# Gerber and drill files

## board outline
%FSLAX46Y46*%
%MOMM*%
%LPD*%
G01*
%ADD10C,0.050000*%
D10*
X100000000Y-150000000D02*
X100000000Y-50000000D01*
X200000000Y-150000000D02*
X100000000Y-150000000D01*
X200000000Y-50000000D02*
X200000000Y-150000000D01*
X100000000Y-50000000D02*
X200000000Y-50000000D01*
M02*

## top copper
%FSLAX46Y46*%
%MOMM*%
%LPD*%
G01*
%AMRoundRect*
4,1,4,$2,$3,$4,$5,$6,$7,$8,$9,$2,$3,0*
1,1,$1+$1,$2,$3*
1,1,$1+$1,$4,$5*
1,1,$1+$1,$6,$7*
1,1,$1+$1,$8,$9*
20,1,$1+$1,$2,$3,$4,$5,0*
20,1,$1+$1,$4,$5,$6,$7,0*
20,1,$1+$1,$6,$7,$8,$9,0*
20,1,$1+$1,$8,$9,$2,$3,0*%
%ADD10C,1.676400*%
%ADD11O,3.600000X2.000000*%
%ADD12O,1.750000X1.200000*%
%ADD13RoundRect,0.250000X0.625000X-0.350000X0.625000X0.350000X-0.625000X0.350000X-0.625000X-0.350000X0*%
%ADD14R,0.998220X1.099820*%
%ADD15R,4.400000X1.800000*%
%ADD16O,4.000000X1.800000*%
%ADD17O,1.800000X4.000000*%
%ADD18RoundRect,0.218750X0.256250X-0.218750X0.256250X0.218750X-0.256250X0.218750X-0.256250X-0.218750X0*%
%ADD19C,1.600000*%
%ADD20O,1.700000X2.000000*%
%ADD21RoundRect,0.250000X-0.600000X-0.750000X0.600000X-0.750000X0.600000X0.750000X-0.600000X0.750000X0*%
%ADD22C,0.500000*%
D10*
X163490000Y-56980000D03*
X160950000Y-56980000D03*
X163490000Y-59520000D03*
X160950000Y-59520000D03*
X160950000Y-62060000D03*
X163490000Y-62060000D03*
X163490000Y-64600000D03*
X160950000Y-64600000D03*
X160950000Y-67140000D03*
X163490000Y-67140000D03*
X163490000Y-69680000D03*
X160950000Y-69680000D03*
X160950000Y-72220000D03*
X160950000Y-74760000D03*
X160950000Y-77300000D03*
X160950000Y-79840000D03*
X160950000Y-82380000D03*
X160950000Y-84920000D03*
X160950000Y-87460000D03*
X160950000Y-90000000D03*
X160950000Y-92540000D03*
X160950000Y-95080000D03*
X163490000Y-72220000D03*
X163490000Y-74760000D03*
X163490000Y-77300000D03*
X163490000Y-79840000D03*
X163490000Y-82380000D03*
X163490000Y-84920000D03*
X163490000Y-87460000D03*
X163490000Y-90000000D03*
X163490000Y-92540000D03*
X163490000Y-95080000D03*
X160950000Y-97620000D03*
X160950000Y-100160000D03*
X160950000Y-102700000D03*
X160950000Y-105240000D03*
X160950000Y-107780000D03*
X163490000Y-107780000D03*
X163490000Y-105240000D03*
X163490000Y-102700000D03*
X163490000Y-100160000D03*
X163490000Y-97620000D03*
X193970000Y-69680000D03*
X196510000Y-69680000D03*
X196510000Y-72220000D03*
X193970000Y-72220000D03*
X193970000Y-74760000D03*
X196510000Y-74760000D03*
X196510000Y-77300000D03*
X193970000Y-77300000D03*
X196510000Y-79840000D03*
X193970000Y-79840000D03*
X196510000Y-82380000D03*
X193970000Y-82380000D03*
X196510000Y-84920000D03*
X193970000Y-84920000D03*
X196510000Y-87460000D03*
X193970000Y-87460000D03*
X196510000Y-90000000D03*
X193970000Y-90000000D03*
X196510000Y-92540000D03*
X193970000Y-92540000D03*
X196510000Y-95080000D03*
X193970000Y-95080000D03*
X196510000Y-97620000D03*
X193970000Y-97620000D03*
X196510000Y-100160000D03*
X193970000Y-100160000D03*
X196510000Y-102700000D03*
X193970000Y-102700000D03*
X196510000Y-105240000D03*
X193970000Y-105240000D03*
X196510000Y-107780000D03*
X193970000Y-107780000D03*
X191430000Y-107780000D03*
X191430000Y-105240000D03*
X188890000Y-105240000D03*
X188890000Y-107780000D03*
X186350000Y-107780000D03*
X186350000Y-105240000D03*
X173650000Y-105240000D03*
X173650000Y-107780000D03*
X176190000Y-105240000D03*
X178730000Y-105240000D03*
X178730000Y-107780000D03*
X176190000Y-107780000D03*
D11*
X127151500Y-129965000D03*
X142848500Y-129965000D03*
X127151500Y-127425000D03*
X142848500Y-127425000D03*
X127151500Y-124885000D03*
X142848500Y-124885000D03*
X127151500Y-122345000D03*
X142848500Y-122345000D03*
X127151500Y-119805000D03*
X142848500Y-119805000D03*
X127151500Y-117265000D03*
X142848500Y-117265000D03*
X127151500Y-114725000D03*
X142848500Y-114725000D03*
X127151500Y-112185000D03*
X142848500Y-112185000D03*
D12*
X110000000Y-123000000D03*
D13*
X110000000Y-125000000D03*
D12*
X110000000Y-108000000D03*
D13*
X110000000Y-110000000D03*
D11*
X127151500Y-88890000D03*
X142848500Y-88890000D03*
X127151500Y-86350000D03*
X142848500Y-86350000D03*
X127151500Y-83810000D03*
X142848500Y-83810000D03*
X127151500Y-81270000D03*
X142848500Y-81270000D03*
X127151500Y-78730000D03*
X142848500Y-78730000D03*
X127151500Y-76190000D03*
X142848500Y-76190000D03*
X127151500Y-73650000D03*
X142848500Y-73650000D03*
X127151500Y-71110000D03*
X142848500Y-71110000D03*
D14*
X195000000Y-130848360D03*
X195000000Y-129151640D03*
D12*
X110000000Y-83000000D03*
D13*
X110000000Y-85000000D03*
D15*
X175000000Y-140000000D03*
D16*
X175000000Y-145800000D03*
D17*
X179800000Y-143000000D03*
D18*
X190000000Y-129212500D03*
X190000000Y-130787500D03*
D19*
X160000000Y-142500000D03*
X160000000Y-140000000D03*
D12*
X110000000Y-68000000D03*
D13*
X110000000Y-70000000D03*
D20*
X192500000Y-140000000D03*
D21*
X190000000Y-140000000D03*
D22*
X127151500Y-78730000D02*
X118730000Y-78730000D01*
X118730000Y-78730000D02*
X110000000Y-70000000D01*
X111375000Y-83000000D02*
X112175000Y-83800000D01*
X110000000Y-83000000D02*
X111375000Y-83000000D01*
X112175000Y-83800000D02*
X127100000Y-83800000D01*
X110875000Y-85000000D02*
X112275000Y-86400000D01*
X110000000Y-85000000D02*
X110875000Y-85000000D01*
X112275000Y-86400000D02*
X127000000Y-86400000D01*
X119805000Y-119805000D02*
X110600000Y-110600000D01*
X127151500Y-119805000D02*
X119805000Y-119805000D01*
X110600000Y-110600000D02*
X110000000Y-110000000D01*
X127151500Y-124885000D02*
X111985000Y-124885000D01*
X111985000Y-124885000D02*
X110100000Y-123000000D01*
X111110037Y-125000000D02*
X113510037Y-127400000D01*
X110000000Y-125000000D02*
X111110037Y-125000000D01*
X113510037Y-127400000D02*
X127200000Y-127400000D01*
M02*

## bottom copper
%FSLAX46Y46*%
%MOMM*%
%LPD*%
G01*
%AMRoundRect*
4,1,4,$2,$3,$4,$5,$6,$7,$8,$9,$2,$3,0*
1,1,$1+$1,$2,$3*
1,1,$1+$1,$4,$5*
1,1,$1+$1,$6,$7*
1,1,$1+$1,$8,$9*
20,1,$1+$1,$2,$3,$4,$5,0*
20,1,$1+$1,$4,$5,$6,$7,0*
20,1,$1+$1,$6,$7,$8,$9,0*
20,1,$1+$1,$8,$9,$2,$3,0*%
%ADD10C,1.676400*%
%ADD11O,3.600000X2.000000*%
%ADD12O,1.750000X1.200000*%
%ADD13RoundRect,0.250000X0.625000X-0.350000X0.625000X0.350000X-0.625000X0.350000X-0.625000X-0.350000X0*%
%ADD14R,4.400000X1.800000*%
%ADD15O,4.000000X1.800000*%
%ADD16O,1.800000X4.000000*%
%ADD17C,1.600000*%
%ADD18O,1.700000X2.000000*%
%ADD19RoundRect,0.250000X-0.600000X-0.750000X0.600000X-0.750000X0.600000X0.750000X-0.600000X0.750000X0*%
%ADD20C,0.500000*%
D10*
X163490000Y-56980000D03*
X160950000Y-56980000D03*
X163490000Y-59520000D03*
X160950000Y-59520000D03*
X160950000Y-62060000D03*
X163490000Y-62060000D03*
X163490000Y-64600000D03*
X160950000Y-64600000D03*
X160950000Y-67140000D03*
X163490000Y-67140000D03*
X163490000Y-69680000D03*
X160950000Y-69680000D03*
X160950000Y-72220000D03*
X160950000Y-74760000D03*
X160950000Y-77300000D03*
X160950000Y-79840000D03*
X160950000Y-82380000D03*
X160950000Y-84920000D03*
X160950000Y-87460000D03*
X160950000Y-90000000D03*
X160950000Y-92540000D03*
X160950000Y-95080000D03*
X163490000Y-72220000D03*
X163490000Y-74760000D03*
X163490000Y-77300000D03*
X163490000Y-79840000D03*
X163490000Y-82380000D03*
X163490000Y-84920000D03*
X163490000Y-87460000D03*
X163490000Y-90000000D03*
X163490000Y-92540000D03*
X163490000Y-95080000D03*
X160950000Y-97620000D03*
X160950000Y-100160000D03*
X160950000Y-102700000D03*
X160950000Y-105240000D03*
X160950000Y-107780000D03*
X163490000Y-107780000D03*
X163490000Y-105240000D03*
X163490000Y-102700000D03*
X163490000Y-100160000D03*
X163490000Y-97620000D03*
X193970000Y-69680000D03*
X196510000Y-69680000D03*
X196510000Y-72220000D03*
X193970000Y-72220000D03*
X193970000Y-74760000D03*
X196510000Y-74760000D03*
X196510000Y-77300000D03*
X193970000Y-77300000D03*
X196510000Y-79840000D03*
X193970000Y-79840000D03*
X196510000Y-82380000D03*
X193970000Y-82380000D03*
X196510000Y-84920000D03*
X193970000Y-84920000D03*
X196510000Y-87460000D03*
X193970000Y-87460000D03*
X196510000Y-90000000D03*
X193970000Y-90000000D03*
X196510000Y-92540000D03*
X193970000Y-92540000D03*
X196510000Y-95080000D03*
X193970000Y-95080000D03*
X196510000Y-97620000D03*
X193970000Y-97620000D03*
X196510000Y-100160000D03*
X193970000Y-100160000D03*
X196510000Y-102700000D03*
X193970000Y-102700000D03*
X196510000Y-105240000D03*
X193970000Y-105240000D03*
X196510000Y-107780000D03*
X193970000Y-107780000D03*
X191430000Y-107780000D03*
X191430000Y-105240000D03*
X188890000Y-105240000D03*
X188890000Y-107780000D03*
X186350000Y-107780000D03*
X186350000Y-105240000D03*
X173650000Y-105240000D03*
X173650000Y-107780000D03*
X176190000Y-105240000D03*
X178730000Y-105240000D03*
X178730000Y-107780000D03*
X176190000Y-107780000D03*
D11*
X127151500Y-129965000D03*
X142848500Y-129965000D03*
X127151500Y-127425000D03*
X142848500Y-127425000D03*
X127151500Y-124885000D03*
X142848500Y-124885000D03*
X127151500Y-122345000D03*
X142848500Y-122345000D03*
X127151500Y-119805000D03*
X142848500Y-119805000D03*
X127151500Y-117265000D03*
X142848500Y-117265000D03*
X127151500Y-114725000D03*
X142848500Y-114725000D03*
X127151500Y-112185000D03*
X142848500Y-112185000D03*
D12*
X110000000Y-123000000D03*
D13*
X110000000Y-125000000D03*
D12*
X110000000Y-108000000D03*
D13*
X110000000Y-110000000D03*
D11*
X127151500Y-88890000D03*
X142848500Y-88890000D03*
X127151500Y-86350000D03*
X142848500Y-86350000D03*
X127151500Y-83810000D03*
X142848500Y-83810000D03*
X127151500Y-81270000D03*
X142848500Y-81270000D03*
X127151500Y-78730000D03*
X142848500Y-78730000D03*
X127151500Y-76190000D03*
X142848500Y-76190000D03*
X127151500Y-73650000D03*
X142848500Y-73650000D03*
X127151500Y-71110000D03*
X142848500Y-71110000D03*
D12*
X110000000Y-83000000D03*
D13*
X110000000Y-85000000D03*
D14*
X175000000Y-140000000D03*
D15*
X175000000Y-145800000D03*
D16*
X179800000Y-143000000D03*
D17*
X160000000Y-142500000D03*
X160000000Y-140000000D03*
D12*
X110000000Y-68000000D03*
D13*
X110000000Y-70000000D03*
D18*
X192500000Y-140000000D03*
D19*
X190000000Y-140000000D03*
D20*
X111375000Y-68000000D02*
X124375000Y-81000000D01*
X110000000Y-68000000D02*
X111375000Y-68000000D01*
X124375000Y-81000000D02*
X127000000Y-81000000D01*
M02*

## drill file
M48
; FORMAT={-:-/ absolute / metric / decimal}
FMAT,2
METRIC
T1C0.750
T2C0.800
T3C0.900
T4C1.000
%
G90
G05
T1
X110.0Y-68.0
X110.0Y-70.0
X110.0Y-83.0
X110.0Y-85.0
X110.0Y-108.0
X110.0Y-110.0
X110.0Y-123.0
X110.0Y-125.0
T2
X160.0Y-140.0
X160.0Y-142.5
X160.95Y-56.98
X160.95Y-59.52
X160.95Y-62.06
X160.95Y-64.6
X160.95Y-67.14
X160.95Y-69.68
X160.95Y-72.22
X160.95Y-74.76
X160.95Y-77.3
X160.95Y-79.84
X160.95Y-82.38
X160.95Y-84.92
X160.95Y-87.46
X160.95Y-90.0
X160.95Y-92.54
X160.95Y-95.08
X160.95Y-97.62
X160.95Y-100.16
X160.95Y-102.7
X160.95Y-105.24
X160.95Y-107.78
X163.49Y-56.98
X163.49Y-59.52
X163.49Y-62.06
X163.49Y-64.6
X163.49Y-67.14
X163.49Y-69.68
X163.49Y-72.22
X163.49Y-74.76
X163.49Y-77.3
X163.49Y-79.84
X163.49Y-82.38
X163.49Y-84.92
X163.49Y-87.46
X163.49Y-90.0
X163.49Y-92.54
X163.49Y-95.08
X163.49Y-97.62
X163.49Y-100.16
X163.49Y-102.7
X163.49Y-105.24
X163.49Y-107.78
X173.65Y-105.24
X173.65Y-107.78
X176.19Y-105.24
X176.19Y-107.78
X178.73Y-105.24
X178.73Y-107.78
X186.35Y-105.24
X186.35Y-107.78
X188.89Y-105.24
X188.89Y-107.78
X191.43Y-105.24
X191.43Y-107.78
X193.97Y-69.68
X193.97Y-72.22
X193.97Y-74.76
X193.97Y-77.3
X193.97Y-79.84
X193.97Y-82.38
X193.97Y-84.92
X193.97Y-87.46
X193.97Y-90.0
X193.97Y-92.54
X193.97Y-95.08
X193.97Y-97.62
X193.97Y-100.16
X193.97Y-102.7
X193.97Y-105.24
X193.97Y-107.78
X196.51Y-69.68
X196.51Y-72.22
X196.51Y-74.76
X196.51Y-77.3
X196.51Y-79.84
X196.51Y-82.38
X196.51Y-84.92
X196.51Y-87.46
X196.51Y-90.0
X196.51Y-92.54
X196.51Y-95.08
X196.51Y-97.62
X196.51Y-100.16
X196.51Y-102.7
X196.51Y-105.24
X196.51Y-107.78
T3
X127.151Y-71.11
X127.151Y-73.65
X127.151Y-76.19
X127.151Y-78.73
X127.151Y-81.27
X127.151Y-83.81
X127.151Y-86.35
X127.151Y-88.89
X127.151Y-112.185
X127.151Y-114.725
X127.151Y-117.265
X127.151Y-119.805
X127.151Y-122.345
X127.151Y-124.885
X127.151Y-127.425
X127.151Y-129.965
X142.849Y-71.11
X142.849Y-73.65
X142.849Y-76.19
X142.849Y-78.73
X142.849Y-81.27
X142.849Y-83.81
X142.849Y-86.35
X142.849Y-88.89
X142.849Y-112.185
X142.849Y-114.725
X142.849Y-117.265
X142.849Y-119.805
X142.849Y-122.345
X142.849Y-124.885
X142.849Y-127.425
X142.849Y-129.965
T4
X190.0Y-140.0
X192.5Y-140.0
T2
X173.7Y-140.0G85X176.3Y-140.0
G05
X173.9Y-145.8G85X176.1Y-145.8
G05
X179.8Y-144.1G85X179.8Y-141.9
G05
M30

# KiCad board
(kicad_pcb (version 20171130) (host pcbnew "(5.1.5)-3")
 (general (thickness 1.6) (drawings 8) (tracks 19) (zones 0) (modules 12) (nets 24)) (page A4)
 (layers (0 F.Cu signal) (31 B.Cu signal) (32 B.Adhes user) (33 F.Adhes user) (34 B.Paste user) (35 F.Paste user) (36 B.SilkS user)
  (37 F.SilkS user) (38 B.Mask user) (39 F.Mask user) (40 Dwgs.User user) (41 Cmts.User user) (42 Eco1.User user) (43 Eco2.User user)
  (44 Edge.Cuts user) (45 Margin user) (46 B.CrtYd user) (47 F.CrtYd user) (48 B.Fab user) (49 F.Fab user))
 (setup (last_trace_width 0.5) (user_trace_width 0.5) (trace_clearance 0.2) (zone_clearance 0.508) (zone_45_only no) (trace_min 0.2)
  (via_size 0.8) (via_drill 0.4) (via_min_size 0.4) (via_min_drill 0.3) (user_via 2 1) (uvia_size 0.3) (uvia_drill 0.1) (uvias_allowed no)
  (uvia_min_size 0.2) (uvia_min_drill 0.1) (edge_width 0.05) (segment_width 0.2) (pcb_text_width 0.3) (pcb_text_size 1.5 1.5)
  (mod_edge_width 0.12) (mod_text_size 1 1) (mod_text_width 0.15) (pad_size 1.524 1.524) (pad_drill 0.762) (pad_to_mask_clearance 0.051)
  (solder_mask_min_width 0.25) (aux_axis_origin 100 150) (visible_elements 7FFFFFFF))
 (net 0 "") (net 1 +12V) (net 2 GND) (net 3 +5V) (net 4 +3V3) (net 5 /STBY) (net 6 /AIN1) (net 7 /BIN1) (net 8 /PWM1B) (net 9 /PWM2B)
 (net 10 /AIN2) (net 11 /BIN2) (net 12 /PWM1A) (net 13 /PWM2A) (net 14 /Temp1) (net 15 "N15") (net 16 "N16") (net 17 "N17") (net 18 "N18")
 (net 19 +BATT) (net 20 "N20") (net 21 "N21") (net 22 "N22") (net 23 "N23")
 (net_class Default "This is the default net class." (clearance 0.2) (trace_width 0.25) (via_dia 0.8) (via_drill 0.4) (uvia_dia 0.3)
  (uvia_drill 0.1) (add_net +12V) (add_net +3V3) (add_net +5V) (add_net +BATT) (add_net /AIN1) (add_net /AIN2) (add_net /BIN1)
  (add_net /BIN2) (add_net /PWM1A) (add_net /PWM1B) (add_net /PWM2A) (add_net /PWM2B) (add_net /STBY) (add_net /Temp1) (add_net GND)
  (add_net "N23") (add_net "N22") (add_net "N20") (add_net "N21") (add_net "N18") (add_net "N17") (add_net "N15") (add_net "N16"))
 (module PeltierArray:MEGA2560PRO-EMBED (layer F.Cu) (at 180 90 270)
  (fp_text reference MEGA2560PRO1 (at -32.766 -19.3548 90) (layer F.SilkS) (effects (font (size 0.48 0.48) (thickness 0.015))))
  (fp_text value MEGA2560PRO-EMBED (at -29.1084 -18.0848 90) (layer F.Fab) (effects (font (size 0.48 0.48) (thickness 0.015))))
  (pad VIN@2 thru_hole circle (at -33.02 16.51 270) (size 1.6764 1.6764) (drill 0.8) (layers *.Cu *.Mask) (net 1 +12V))
  (pad VIN@1 thru_hole circle (at -33.02 19.05 270) (size 1.6764 1.6764) (drill 0.8) (layers *.Cu *.Mask) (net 1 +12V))
  (pad GND@2 thru_hole circle (at -30.48 16.51 270) (size 1.6764 1.6764) (drill 0.8) (layers *.Cu *.Mask) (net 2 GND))
  (pad GND@1 thru_hole circle (at -30.48 19.05 270) (size 1.6764 1.6764) (drill 0.8) (layers *.Cu *.Mask) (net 2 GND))
  (pad 5V@1 thru_hole circle (at -27.94 19.05 270) (size 1.6764 1.6764) (drill 0.8) (layers *.Cu *.Mask) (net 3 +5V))
  (pad 5V@2 thru_hole circle (at -27.94 16.51 270) (size 1.6764 1.6764) (drill 0.8) (layers *.Cu *.Mask) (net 3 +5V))
  (pad 3V3@2 thru_hole circle (at -25.4 16.51 270) (size 1.6764 1.6764) (drill 0.8) (layers *.Cu *.Mask) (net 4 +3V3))
  (pad 3V3@1 thru_hole circle (at -25.4 19.05 270) (size 1.6764 1.6764) (drill 0.8) (layers *.Cu *.Mask) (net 4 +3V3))
  (pad RST thru_hole circle (at -22.86 19.05 270) (size 1.6764 1.6764) (drill 0.8) (layers *.Cu *.Mask))
  (pad AREF thru_hole circle (at -22.86 16.51 270) (size 1.6764 1.6764) (drill 0.8) (layers *.Cu *.Mask))
  (pad RX thru_hole circle (at -20.32 16.51 270) (size 1.6764 1.6764) (drill 0.8) (layers *.Cu *.Mask))
  (pad TX thru_hole circle (at -20.32 19.05 270) (size 1.6764 1.6764) (drill 0.8) (layers *.Cu *.Mask))
  (pad D3 thru_hole circle (at -17.78 19.05 270) (size 1.6764 1.6764) (drill 0.8) (layers *.Cu *.Mask) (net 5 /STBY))
  (pad D5 thru_hole circle (at -15.24 19.05 270) (size 1.6764 1.6764) (drill 0.8) (layers *.Cu *.Mask) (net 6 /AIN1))
  (pad D7 thru_hole circle (at -12.7 19.05 270) (size 1.6764 1.6764) (drill 0.8) (layers *.Cu *.Mask) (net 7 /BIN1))
  (pad D9 thru_hole circle (at -10.16 19.05 270) (size 1.6764 1.6764) (drill 0.8) (layers *.Cu *.Mask) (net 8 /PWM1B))
  (pad D11 thru_hole circle (at -7.62 19.05 270) (size 1.6764 1.6764) (drill 0.8) (layers *.Cu *.Mask) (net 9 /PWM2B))
  (pad D13 thru_hole circle (at -5.08 19.05 270) (size 1.6764 1.6764) (drill 0.8) (layers *.Cu *.Mask))
  (pad D15 thru_hole circle (at -2.54 19.05 270) (size 1.6764 1.6764) (drill 0.8) (layers *.Cu *.Mask))
  (pad D17 thru_hole circle (at 0 19.05 270) (size 1.6764 1.6764) (drill 0.8) (layers *.Cu *.Mask))
  (pad D19 thru_hole circle (at 2.54 19.05 270) (size 1.6764 1.6764) (drill 0.8) (layers *.Cu *.Mask))
  (pad D21 thru_hole circle (at 5.08 19.05 270) (size 1.6764 1.6764) (drill 0.8) (layers *.Cu *.Mask))
  (pad D2 thru_hole circle (at -17.78 16.51 270) (size 1.6764 1.6764) (drill 0.8) (layers *.Cu *.Mask))
  (pad D4 thru_hole circle (at -15.24 16.51 270) (size 1.6764 1.6764) (drill 0.8) (layers *.Cu *.Mask) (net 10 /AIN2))
  (pad D6 thru_hole circle (at -12.7 16.51 270) (size 1.6764 1.6764) (drill 0.8) (layers *.Cu *.Mask) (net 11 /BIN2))
  (pad D8 thru_hole circle (at -10.16 16.51 270) (size 1.6764 1.6764) (drill 0.8) (layers *.Cu *.Mask) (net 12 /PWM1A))
  (pad D10 thru_hole circle (at -7.62 16.51 270) (size 1.6764 1.6764) (drill 0.8) (layers *.Cu *.Mask) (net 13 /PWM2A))
  (pad D12 thru_hole circle (at -5.08 16.51 270) (size 1.6764 1.6764) (drill 0.8) (layers *.Cu *.Mask))
  (pad D14 thru_hole circle (at -2.54 16.51 270) (size 1.6764 1.6764) (drill 0.8) (layers *.Cu *.Mask))
  (pad D16 thru_hole circle (at 0 16.51 270) (size 1.6764 1.6764) (drill 0.8) (layers *.Cu *.Mask))
  (pad D18 thru_hole circle (at 2.54 16.51 270) (size 1.6764 1.6764) (drill 0.8) (layers *.Cu *.Mask))
  (pad D20 thru_hole circle (at 5.08 16.51 270) (size 1.6764 1.6764) (drill 0.8) (layers *.Cu *.Mask))
  (pad D23 thru_hole circle (at 7.62 19.05 270) (size 1.6764 1.6764) (drill 0.8) (layers *.Cu *.Mask))
  (pad D25 thru_hole circle (at 10.16 19.05 270) (size 1.6764 1.6764) (drill 0.8) (layers *.Cu *.Mask))
  (pad D27 thru_hole circle (at 12.7 19.05 270) (size 1.6764 1.6764) (drill 0.8) (layers *.Cu *.Mask))
  (pad D29 thru_hole circle (at 15.24 19.05 270) (size 1.6764 1.6764) (drill 0.8) (layers *.Cu *.Mask))
  (pad D31 thru_hole circle (at 17.78 19.05 270) (size 1.6764 1.6764) (drill 0.8) (layers *.Cu *.Mask))
  (pad D30 thru_hole circle (at 17.78 16.51 270) (size 1.6764 1.6764) (drill 0.8) (layers *.Cu *.Mask))
  (pad D28 thru_hole circle (at 15.24 16.51 270) (size 1.6764 1.6764) (drill 0.8) (layers *.Cu *.Mask))
  (pad D26 thru_hole circle (at 12.7 16.51 270) (size 1.6764 1.6764) (drill 0.8) (layers *.Cu *.Mask))
  (pad D24 thru_hole circle (at 10.16 16.51 270) (size 1.6764 1.6764) (drill 0.8) (layers *.Cu *.Mask))
  (pad D22 thru_hole circle (at 7.62 16.51 270) (size 1.6764 1.6764) (drill 0.8) (layers *.Cu *.Mask))
  (pad A1 thru_hole circle (at -20.32 -13.97 270) (size 1.6764 1.6764) (drill 0.8) (layers *.Cu *.Mask))
  (pad A0 thru_hole circle (at -20.32 -16.51 270) (size 1.6764 1.6764) (drill 0.8) (layers *.Cu *.Mask) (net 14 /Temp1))
  (pad A2 thru_hole circle (at -17.78 -16.51 270) (size 1.6764 1.6764) (drill 0.8) (layers *.Cu *.Mask))
  (pad A3 thru_hole circle (at -17.78 -13.97 270) (size 1.6764 1.6764) (drill 0.8) (layers *.Cu *.Mask))
  (pad A5 thru_hole circle (at -15.24 -13.97 270) (size 1.6764 1.6764) (drill 0.8) (layers *.Cu *.Mask))
  (pad A4 thru_hole circle (at -15.24 -16.51 270) (size 1.6764 1.6764) (drill 0.8) (layers *.Cu *.Mask))
  (pad A6 thru_hole circle (at -12.7 -16.51 270) (size 1.6764 1.6764) (drill 0.8) (layers *.Cu *.Mask))
  (pad A7 thru_hole circle (at -12.7 -13.97 270) (size 1.6764 1.6764) (drill 0.8) (layers *.Cu *.Mask))
  (pad A8 thru_hole circle (at -10.16 -16.51 270) (size 1.6764 1.6764) (drill 0.8) (layers *.Cu *.Mask))
  (pad A9 thru_hole circle (at -10.16 -13.97 270) (size 1.6764 1.6764) (drill 0.8) (layers *.Cu *.Mask))
  (pad A10 thru_hole circle (at -7.62 -16.51 270) (size 1.6764 1.6764) (drill 0.8) (layers *.Cu *.Mask))
  (pad A11 thru_hole circle (at -7.62 -13.97 270) (size 1.6764 1.6764) (drill 0.8) (layers *.Cu *.Mask))
  (pad A12 thru_hole circle (at -5.08 -16.51 270) (size 1.6764 1.6764) (drill 0.8) (layers *.Cu *.Mask))
  (pad A13 thru_hole circle (at -5.08 -13.97 270) (size 1.6764 1.6764) (drill 0.8) (layers *.Cu *.Mask))
  (pad A14 thru_hole circle (at -2.54 -16.51 270) (size 1.6764 1.6764) (drill 0.8) (layers *.Cu *.Mask))
  (pad A15 thru_hole circle (at -2.54 -13.97 270) (size 1.6764 1.6764) (drill 0.8) (layers *.Cu *.Mask))
  (pad D32 thru_hole circle (at 0 -16.51 270) (size 1.6764 1.6764) (drill 0.8) (layers *.Cu *.Mask))
  (pad D33 thru_hole circle (at 0 -13.97 270) (size 1.6764 1.6764) (drill 0.8) (layers *.Cu *.Mask))
  (pad D34 thru_hole circle (at 2.54 -16.51 270) (size 1.6764 1.6764) (drill 0.8) (layers *.Cu *.Mask))
  (pad D35 thru_hole circle (at 2.54 -13.97 270) (size 1.6764 1.6764) (drill 0.8) (layers *.Cu *.Mask))
  (pad D36 thru_hole circle (at 5.08 -16.51 270) (size 1.6764 1.6764) (drill 0.8) (layers *.Cu *.Mask))
  (pad D37 thru_hole circle (at 5.08 -13.97 270) (size 1.6764 1.6764) (drill 0.8) (layers *.Cu *.Mask))
  (pad D38 thru_hole circle (at 7.62 -16.51 270) (size 1.6764 1.6764) (drill 0.8) (layers *.Cu *.Mask))
  (pad D39 thru_hole circle (at 7.62 -13.97 270) (size 1.6764 1.6764) (drill 0.8) (layers *.Cu *.Mask))
  (pad D40 thru_hole circle (at 10.16 -16.51 270) (size 1.6764 1.6764) (drill 0.8) (layers *.Cu *.Mask))
  (pad D41 thru_hole circle (at 10.16 -13.97 270) (size 1.6764 1.6764) (drill 0.8) (layers *.Cu *.Mask))
  (pad D42 thru_hole circle (at 12.7 -16.51 270) (size 1.6764 1.6764) (drill 0.8) (layers *.Cu *.Mask))
  (pad D43 thru_hole circle (at 12.7 -13.97 270) (size 1.6764 1.6764) (drill 0.8) (layers *.Cu *.Mask))
  (pad D44 thru_hole circle (at 15.24 -16.51 270) (size 1.6764 1.6764) (drill 0.8) (layers *.Cu *.Mask))
  (pad D45 thru_hole circle (at 15.24 -13.97 270) (size 1.6764 1.6764) (drill 0.8) (layers *.Cu *.Mask))
  (pad D46 thru_hole circle (at 17.78 -16.51 270) (size 1.6764 1.6764) (drill 0.8) (layers *.Cu *.Mask))
  (pad D47 thru_hole circle (at 17.78 -13.97 270) (size 1.6764 1.6764) (drill 0.8) (layers *.Cu *.Mask))
  (pad D48 thru_hole circle (at 17.78 -11.43 270) (size 1.6764 1.6764) (drill 0.8) (layers *.Cu *.Mask))
  (pad D49 thru_hole circle (at 15.24 -11.43 270) (size 1.6764 1.6764) (drill 0.8) (layers *.Cu *.Mask))
  (pad D51 thru_hole circle (at 15.24 -8.89 270) (size 1.6764 1.6764) (drill 0.8) (layers *.Cu *.Mask))
  (pad D50 thru_hole circle (at 17.78 -8.89 270) (size 1.6764 1.6764) (drill 0.8) (layers *.Cu *.Mask))
  (pad D52 thru_hole circle (at 17.78 -6.35 270) (size 1.6764 1.6764) (drill 0.8) (layers *.Cu *.Mask))
  (pad D53 thru_hole circle (at 15.24 -6.35 270) (size 1.6764 1.6764) (drill 0.8) (layers *.Cu *.Mask))
  (pad RESET thru_hole circle (at 15.24 6.35 270) (size 1.6764 1.6764) (drill 0.8) (layers *.Cu *.Mask))
  (pad GND@3 thru_hole circle (at 17.78 6.35 270) (size 1.6764 1.6764) (drill 0.8) (layers *.Cu *.Mask) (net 2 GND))
  (pad SCK thru_hole circle (at 15.24 3.81 270) (size 1.6764 1.6764) (drill 0.8) (layers *.Cu *.Mask))
  (pad MISO thru_hole circle (at 15.24 1.27 270) (size 1.6764 1.6764) (drill 0.8) (layers *.Cu *.Mask))
  (pad 5V@3 thru_hole circle (at 17.78 1.27 270) (size 1.6764 1.6764) (drill 0.8) (layers *.Cu *.Mask) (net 3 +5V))
  (pad MOSI thru_hole circle (at 17.78 3.81 270) (size 1.6764 1.6764) (drill 0.8) (layers *.Cu *.Mask)))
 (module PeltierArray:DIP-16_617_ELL (layer F.Cu) (at 135 121.075 270)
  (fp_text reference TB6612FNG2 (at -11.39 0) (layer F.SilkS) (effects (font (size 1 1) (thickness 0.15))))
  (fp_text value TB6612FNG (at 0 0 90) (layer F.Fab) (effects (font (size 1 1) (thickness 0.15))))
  (pad 8 thru_hole oval (at 8.89 7.8485 270) (size 2 3.6) (drill 0.9) (layers *.Cu *.Mask) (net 2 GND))
  (pad 9 thru_hole oval (at 8.89 -7.8485 270) (size 2 3.6) (drill 0.9) (layers *.Cu *.Mask) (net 13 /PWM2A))
  (pad 7 thru_hole oval (at 6.35 7.8485 270) (size 2 3.6) (drill 0.9) (layers *.Cu *.Mask) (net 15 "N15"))
  (pad 10 thru_hole oval (at 6.35 -7.8485 270) (size 2 3.6) (drill 0.9) (layers *.Cu *.Mask) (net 10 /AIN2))
  (pad 6 thru_hole oval (at 3.81 7.8485 270) (size 2 3.6) (drill 0.9) (layers *.Cu *.Mask) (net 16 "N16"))
  (pad 11 thru_hole oval (at 3.81 -7.8485 270) (size 2 3.6) (drill 0.9) (layers *.Cu *.Mask) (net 6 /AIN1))
  (pad 5 thru_hole oval (at 1.27 7.8485 270) (size 2 3.6) (drill 0.9) (layers *.Cu *.Mask) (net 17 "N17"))
  (pad 12 thru_hole oval (at 1.27 -7.8485 270) (size 2 3.6) (drill 0.9) (layers *.Cu *.Mask) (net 5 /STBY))
  (pad 4 thru_hole oval (at -1.27 7.8485 270) (size 2 3.6) (drill 0.9) (layers *.Cu *.Mask) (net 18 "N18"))
  (pad 13 thru_hole oval (at -1.27 -7.8485 270) (size 2 3.6) (drill 0.9) (layers *.Cu *.Mask) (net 7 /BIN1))
  (pad 3 thru_hole oval (at -3.81 7.8485 270) (size 2 3.6) (drill 0.9) (layers *.Cu *.Mask) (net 2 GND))
  (pad 14 thru_hole oval (at -3.81 -7.8485 270) (size 2 3.6) (drill 0.9) (layers *.Cu *.Mask) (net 11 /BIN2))
  (pad 2 thru_hole oval (at -6.35 7.8485 270) (size 2 3.6) (drill 0.9) (layers *.Cu *.Mask) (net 3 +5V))
  (pad 15 thru_hole oval (at -6.35 -7.8485 270) (size 2 3.6) (drill 0.9) (layers *.Cu *.Mask) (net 9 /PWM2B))
  (pad 1 thru_hole oval (at -8.89 7.8485 270) (size 2 3.6) (drill 0.9) (layers *.Cu *.Mask) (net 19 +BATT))
  (pad 16 thru_hole oval (at -8.89 -7.8485 270) (size 2 3.6) (drill 0.9) (layers *.Cu *.Mask) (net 2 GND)))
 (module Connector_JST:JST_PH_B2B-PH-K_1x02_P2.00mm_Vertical (layer F.Cu) (at 110 125 90)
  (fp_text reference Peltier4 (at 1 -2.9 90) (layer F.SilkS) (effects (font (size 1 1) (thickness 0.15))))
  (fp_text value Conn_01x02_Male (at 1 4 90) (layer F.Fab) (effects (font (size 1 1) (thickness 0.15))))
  (pad 2 thru_hole oval (at 2 0 90) (size 1.2 1.75) (drill 0.75) (layers *.Cu *.Mask) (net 16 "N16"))
  (pad 1 thru_hole roundrect (at 0 0 90) (size 1.2 1.75) (drill 0.75) (layers *.Cu *.Mask) (roundrect_rratio 0.208333) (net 15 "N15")))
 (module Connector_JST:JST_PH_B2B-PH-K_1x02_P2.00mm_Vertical (layer F.Cu) (at 110 110 90)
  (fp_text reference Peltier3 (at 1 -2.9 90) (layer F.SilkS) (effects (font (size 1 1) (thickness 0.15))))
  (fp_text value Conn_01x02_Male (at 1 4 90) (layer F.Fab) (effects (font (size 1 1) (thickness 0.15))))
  (pad 2 thru_hole oval (at 2 0 90) (size 1.2 1.75) (drill 0.75) (layers *.Cu *.Mask) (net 17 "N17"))
  (pad 1 thru_hole roundrect (at 0 0 90) (size 1.2 1.75) (drill 0.75) (layers *.Cu *.Mask) (roundrect_rratio 0.208333) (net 18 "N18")))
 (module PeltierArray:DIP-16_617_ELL (layer F.Cu) (at 135 80 270)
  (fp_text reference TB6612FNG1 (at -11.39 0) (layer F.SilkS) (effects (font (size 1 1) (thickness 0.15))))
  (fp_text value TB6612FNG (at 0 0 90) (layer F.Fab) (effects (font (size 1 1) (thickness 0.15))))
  (pad 8 thru_hole oval (at 8.89 7.8485 270) (size 2 3.6) (drill 0.9) (layers *.Cu *.Mask) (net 2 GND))
  (pad 9 thru_hole oval (at 8.89 -7.8485 270) (size 2 3.6) (drill 0.9) (layers *.Cu *.Mask) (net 12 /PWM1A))
  (pad 7 thru_hole oval (at 6.35 7.8485 270) (size 2 3.6) (drill 0.9) (layers *.Cu *.Mask) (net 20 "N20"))
  (pad 10 thru_hole oval (at 6.35 -7.8485 270) (size 2 3.6) (drill 0.9) (layers *.Cu *.Mask) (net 10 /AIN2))
  (pad 6 thru_hole oval (at 3.81 7.8485 270) (size 2 3.6) (drill 0.9) (layers *.Cu *.Mask) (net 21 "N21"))
  (pad 11 thru_hole oval (at 3.81 -7.8485 270) (size 2 3.6) (drill 0.9) (layers *.Cu *.Mask) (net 6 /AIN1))
  (pad 5 thru_hole oval (at 1.27 7.8485 270) (size 2 3.6) (drill 0.9) (layers *.Cu *.Mask) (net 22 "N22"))
  (pad 12 thru_hole oval (at 1.27 -7.8485 270) (size 2 3.6) (drill 0.9) (layers *.Cu *.Mask) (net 5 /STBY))
  (pad 4 thru_hole oval (at -1.27 7.8485 270) (size 2 3.6) (drill 0.9) (layers *.Cu *.Mask) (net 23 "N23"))
  (pad 13 thru_hole oval (at -1.27 -7.8485 270) (size 2 3.6) (drill 0.9) (layers *.Cu *.Mask) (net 7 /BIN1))
  (pad 3 thru_hole oval (at -3.81 7.8485 270) (size 2 3.6) (drill 0.9) (layers *.Cu *.Mask) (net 2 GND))
  (pad 14 thru_hole oval (at -3.81 -7.8485 270) (size 2 3.6) (drill 0.9) (layers *.Cu *.Mask) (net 11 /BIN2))
  (pad 2 thru_hole oval (at -6.35 7.8485 270) (size 2 3.6) (drill 0.9) (layers *.Cu *.Mask) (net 3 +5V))
  (pad 15 thru_hole oval (at -6.35 -7.8485 270) (size 2 3.6) (drill 0.9) (layers *.Cu *.Mask) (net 8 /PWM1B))
  (pad 1 thru_hole oval (at -8.89 7.8485 270) (size 2 3.6) (drill 0.9) (layers *.Cu *.Mask) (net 19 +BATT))
  (pad 16 thru_hole oval (at -8.89 -7.8485 270) (size 2 3.6) (drill 0.9) (layers *.Cu *.Mask) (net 2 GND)))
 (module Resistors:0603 (layer F.Cu) (at 195 130 270)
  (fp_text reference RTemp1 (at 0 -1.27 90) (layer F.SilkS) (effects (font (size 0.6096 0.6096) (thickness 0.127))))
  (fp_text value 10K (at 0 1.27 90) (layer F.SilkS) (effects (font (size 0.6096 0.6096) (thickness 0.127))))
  (pad 2 smd rect (at 0.84836 0 270) (size 1.09982 0.99822) (layers F.Cu F.Paste F.Mask) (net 14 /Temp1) (solder_mask_margin 0.1016))
  (pad 1 smd rect (at -0.84836 0 270) (size 1.09982 0.99822) (layers F.Cu F.Paste F.Mask) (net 2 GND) (solder_mask_margin 0.1016)))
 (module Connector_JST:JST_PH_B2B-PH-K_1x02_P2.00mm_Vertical (layer F.Cu) (at 110 85 90)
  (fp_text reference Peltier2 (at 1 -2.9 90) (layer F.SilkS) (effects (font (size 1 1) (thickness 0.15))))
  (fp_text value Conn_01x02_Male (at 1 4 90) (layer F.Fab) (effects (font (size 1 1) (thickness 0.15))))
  (pad 2 thru_hole oval (at 2 0 90) (size 1.2 1.75) (drill 0.75) (layers *.Cu *.Mask) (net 21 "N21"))
  (pad 1 thru_hole roundrect (at 0 0 90) (size 1.2 1.75) (drill 0.75) (layers *.Cu *.Mask) (roundrect_rratio 0.208333) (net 20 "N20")))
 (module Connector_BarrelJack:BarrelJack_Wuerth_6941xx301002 (layer F.Cu) (at 175 140)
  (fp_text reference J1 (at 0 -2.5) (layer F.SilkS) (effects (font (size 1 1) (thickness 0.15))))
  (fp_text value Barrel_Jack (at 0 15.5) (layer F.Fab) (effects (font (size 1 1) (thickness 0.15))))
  (pad 1 thru_hole rect (at 0 0) (size 4.4 1.8) (drill oval 3.4 0.8) (layers *.Cu *.Mask) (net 19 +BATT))
  (pad 2 thru_hole oval (at 0 5.8) (size 4 1.8) (drill oval 3 0.8) (layers *.Cu *.Mask) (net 2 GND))
  (pad 3 thru_hole oval (at 4.8 3 90) (size 4 1.8) (drill oval 3 0.8) (layers *.Cu *.Mask)))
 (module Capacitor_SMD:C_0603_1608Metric (layer F.Cu) (at 190 130 90)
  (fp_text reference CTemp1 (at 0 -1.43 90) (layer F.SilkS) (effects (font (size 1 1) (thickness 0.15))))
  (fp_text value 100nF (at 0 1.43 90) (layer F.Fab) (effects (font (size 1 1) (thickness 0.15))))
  (pad 2 smd roundrect (at 0.7875 0 90) (size 0.875 0.95) (layers F.Cu F.Paste F.Mask) (roundrect_rratio 0.25) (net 2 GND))
  (pad 1 smd roundrect (at -0.7875 0 90) (size 0.875 0.95) (layers F.Cu F.Paste F.Mask) (roundrect_rratio 0.25) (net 3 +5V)))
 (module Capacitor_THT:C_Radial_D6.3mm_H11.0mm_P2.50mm (layer F.Cu) (at 160 140 270)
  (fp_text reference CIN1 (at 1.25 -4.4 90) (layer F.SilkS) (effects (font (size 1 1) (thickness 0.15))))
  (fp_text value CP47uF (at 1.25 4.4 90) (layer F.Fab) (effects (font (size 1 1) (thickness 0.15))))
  (pad 2 thru_hole circle (at 2.5 0 270) (size 1.6 1.6) (drill 0.8) (layers *.Cu *.Mask) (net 2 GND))
  (pad 1 thru_hole circle (at 0 0 270) (size 1.6 1.6) (drill 0.8) (layers *.Cu *.Mask) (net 19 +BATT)))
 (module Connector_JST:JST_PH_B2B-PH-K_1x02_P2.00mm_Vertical (layer F.Cu) (at 110 70 90)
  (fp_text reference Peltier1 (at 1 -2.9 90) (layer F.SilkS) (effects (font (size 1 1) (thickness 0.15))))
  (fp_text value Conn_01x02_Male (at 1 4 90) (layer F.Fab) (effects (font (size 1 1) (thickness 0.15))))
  (pad 2 thru_hole oval (at 2 0 90) (size 1.2 1.75) (drill 0.75) (layers *.Cu *.Mask) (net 22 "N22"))
  (pad 1 thru_hole roundrect (at 0 0 90) (size 1.2 1.75) (drill 0.75) (layers *.Cu *.Mask) (roundrect_rratio 0.208333) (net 23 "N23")))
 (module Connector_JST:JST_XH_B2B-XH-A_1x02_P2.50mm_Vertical (layer F.Cu) (at 190 140)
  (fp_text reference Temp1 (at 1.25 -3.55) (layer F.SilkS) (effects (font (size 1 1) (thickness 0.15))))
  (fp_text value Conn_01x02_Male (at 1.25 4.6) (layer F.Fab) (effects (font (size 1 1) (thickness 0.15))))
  (pad 2 thru_hole oval (at 2.5 0) (size 1.7 2) (drill 1) (layers *.Cu *.Mask) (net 14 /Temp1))
  (pad 1 thru_hole roundrect (at 0 0) (size 1.7 2) (drill 1) (layers *.Cu *.Mask) (roundrect_rratio 0.147059) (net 3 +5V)))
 (gr_line (start 100 150) (end 100 50) (layer Edge.Cuts) (width 0.05))
 (gr_line (start 200 150) (end 100 150) (layer Edge.Cuts) (width 0.05))
 (gr_line (start 200 50) (end 200 150) (layer Edge.Cuts) (width 0.05))
 (gr_line (start 100 50) (end 200 50) (layer Edge.Cuts) (width 0.05))
 (segment (start 111.375 68) (end 124.375 81) (width 0.5) (layer B.Cu) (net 22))
 (segment (start 110 68) (end 111.375 68) (width 0.5) (layer B.Cu) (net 22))
 (segment (start 124.375 81) (end 127 81) (width 0.5) (layer B.Cu) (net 22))
 (segment (start 127.1515 78.73) (end 118.73 78.73) (width 0.5) (layer F.Cu) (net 23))
 (segment (start 118.73 78.73) (end 110 70) (width 0.5) (layer F.Cu) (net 23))
 (segment (start 111.375 83) (end 112.175 83.8) (width 0.5) (layer F.Cu) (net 21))
 (segment (start 110 83) (end 111.375 83) (width 0.5) (layer F.Cu) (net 21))
 (segment (start 112.175 83.8) (end 127.1 83.8) (width 0.5) (layer F.Cu) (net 21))
 (segment (start 110.875 85) (end 112.275 86.4) (width 0.5) (layer F.Cu) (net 20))
 (segment (start 110 85) (end 110.875 85) (width 0.5) (layer F.Cu) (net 20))
 (segment (start 112.275 86.4) (end 127 86.4) (width 0.5) (layer F.Cu) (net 20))
 (segment (start 119.805 119.805) (end 110.6 110.6) (width 0.5) (layer F.Cu) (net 18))
 (segment (start 127.1515 119.805) (end 119.805 119.805) (width 0.5) (layer F.Cu) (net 18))
 (segment (start 110.6 110.6) (end 110 110) (width 0.5) (layer F.Cu) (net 18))
 (segment (start 127.1515 124.885) (end 111.985 124.885) (width 0.5) (layer F.Cu) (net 16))
 (segment (start 111.985 124.885) (end 110.1 123) (width 0.5) (layer F.Cu) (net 16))
 (segment (start 111.110037 125) (end 113.510037 127.4) (width 0.5) (layer F.Cu) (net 15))
 (segment (start 110 125) (end 111.110037 125) (width 0.5) (layer F.Cu) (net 15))
 (segment (start 113.510037 127.4) (end 127.2 127.4) (width 0.5) (layer F.Cu) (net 15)))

